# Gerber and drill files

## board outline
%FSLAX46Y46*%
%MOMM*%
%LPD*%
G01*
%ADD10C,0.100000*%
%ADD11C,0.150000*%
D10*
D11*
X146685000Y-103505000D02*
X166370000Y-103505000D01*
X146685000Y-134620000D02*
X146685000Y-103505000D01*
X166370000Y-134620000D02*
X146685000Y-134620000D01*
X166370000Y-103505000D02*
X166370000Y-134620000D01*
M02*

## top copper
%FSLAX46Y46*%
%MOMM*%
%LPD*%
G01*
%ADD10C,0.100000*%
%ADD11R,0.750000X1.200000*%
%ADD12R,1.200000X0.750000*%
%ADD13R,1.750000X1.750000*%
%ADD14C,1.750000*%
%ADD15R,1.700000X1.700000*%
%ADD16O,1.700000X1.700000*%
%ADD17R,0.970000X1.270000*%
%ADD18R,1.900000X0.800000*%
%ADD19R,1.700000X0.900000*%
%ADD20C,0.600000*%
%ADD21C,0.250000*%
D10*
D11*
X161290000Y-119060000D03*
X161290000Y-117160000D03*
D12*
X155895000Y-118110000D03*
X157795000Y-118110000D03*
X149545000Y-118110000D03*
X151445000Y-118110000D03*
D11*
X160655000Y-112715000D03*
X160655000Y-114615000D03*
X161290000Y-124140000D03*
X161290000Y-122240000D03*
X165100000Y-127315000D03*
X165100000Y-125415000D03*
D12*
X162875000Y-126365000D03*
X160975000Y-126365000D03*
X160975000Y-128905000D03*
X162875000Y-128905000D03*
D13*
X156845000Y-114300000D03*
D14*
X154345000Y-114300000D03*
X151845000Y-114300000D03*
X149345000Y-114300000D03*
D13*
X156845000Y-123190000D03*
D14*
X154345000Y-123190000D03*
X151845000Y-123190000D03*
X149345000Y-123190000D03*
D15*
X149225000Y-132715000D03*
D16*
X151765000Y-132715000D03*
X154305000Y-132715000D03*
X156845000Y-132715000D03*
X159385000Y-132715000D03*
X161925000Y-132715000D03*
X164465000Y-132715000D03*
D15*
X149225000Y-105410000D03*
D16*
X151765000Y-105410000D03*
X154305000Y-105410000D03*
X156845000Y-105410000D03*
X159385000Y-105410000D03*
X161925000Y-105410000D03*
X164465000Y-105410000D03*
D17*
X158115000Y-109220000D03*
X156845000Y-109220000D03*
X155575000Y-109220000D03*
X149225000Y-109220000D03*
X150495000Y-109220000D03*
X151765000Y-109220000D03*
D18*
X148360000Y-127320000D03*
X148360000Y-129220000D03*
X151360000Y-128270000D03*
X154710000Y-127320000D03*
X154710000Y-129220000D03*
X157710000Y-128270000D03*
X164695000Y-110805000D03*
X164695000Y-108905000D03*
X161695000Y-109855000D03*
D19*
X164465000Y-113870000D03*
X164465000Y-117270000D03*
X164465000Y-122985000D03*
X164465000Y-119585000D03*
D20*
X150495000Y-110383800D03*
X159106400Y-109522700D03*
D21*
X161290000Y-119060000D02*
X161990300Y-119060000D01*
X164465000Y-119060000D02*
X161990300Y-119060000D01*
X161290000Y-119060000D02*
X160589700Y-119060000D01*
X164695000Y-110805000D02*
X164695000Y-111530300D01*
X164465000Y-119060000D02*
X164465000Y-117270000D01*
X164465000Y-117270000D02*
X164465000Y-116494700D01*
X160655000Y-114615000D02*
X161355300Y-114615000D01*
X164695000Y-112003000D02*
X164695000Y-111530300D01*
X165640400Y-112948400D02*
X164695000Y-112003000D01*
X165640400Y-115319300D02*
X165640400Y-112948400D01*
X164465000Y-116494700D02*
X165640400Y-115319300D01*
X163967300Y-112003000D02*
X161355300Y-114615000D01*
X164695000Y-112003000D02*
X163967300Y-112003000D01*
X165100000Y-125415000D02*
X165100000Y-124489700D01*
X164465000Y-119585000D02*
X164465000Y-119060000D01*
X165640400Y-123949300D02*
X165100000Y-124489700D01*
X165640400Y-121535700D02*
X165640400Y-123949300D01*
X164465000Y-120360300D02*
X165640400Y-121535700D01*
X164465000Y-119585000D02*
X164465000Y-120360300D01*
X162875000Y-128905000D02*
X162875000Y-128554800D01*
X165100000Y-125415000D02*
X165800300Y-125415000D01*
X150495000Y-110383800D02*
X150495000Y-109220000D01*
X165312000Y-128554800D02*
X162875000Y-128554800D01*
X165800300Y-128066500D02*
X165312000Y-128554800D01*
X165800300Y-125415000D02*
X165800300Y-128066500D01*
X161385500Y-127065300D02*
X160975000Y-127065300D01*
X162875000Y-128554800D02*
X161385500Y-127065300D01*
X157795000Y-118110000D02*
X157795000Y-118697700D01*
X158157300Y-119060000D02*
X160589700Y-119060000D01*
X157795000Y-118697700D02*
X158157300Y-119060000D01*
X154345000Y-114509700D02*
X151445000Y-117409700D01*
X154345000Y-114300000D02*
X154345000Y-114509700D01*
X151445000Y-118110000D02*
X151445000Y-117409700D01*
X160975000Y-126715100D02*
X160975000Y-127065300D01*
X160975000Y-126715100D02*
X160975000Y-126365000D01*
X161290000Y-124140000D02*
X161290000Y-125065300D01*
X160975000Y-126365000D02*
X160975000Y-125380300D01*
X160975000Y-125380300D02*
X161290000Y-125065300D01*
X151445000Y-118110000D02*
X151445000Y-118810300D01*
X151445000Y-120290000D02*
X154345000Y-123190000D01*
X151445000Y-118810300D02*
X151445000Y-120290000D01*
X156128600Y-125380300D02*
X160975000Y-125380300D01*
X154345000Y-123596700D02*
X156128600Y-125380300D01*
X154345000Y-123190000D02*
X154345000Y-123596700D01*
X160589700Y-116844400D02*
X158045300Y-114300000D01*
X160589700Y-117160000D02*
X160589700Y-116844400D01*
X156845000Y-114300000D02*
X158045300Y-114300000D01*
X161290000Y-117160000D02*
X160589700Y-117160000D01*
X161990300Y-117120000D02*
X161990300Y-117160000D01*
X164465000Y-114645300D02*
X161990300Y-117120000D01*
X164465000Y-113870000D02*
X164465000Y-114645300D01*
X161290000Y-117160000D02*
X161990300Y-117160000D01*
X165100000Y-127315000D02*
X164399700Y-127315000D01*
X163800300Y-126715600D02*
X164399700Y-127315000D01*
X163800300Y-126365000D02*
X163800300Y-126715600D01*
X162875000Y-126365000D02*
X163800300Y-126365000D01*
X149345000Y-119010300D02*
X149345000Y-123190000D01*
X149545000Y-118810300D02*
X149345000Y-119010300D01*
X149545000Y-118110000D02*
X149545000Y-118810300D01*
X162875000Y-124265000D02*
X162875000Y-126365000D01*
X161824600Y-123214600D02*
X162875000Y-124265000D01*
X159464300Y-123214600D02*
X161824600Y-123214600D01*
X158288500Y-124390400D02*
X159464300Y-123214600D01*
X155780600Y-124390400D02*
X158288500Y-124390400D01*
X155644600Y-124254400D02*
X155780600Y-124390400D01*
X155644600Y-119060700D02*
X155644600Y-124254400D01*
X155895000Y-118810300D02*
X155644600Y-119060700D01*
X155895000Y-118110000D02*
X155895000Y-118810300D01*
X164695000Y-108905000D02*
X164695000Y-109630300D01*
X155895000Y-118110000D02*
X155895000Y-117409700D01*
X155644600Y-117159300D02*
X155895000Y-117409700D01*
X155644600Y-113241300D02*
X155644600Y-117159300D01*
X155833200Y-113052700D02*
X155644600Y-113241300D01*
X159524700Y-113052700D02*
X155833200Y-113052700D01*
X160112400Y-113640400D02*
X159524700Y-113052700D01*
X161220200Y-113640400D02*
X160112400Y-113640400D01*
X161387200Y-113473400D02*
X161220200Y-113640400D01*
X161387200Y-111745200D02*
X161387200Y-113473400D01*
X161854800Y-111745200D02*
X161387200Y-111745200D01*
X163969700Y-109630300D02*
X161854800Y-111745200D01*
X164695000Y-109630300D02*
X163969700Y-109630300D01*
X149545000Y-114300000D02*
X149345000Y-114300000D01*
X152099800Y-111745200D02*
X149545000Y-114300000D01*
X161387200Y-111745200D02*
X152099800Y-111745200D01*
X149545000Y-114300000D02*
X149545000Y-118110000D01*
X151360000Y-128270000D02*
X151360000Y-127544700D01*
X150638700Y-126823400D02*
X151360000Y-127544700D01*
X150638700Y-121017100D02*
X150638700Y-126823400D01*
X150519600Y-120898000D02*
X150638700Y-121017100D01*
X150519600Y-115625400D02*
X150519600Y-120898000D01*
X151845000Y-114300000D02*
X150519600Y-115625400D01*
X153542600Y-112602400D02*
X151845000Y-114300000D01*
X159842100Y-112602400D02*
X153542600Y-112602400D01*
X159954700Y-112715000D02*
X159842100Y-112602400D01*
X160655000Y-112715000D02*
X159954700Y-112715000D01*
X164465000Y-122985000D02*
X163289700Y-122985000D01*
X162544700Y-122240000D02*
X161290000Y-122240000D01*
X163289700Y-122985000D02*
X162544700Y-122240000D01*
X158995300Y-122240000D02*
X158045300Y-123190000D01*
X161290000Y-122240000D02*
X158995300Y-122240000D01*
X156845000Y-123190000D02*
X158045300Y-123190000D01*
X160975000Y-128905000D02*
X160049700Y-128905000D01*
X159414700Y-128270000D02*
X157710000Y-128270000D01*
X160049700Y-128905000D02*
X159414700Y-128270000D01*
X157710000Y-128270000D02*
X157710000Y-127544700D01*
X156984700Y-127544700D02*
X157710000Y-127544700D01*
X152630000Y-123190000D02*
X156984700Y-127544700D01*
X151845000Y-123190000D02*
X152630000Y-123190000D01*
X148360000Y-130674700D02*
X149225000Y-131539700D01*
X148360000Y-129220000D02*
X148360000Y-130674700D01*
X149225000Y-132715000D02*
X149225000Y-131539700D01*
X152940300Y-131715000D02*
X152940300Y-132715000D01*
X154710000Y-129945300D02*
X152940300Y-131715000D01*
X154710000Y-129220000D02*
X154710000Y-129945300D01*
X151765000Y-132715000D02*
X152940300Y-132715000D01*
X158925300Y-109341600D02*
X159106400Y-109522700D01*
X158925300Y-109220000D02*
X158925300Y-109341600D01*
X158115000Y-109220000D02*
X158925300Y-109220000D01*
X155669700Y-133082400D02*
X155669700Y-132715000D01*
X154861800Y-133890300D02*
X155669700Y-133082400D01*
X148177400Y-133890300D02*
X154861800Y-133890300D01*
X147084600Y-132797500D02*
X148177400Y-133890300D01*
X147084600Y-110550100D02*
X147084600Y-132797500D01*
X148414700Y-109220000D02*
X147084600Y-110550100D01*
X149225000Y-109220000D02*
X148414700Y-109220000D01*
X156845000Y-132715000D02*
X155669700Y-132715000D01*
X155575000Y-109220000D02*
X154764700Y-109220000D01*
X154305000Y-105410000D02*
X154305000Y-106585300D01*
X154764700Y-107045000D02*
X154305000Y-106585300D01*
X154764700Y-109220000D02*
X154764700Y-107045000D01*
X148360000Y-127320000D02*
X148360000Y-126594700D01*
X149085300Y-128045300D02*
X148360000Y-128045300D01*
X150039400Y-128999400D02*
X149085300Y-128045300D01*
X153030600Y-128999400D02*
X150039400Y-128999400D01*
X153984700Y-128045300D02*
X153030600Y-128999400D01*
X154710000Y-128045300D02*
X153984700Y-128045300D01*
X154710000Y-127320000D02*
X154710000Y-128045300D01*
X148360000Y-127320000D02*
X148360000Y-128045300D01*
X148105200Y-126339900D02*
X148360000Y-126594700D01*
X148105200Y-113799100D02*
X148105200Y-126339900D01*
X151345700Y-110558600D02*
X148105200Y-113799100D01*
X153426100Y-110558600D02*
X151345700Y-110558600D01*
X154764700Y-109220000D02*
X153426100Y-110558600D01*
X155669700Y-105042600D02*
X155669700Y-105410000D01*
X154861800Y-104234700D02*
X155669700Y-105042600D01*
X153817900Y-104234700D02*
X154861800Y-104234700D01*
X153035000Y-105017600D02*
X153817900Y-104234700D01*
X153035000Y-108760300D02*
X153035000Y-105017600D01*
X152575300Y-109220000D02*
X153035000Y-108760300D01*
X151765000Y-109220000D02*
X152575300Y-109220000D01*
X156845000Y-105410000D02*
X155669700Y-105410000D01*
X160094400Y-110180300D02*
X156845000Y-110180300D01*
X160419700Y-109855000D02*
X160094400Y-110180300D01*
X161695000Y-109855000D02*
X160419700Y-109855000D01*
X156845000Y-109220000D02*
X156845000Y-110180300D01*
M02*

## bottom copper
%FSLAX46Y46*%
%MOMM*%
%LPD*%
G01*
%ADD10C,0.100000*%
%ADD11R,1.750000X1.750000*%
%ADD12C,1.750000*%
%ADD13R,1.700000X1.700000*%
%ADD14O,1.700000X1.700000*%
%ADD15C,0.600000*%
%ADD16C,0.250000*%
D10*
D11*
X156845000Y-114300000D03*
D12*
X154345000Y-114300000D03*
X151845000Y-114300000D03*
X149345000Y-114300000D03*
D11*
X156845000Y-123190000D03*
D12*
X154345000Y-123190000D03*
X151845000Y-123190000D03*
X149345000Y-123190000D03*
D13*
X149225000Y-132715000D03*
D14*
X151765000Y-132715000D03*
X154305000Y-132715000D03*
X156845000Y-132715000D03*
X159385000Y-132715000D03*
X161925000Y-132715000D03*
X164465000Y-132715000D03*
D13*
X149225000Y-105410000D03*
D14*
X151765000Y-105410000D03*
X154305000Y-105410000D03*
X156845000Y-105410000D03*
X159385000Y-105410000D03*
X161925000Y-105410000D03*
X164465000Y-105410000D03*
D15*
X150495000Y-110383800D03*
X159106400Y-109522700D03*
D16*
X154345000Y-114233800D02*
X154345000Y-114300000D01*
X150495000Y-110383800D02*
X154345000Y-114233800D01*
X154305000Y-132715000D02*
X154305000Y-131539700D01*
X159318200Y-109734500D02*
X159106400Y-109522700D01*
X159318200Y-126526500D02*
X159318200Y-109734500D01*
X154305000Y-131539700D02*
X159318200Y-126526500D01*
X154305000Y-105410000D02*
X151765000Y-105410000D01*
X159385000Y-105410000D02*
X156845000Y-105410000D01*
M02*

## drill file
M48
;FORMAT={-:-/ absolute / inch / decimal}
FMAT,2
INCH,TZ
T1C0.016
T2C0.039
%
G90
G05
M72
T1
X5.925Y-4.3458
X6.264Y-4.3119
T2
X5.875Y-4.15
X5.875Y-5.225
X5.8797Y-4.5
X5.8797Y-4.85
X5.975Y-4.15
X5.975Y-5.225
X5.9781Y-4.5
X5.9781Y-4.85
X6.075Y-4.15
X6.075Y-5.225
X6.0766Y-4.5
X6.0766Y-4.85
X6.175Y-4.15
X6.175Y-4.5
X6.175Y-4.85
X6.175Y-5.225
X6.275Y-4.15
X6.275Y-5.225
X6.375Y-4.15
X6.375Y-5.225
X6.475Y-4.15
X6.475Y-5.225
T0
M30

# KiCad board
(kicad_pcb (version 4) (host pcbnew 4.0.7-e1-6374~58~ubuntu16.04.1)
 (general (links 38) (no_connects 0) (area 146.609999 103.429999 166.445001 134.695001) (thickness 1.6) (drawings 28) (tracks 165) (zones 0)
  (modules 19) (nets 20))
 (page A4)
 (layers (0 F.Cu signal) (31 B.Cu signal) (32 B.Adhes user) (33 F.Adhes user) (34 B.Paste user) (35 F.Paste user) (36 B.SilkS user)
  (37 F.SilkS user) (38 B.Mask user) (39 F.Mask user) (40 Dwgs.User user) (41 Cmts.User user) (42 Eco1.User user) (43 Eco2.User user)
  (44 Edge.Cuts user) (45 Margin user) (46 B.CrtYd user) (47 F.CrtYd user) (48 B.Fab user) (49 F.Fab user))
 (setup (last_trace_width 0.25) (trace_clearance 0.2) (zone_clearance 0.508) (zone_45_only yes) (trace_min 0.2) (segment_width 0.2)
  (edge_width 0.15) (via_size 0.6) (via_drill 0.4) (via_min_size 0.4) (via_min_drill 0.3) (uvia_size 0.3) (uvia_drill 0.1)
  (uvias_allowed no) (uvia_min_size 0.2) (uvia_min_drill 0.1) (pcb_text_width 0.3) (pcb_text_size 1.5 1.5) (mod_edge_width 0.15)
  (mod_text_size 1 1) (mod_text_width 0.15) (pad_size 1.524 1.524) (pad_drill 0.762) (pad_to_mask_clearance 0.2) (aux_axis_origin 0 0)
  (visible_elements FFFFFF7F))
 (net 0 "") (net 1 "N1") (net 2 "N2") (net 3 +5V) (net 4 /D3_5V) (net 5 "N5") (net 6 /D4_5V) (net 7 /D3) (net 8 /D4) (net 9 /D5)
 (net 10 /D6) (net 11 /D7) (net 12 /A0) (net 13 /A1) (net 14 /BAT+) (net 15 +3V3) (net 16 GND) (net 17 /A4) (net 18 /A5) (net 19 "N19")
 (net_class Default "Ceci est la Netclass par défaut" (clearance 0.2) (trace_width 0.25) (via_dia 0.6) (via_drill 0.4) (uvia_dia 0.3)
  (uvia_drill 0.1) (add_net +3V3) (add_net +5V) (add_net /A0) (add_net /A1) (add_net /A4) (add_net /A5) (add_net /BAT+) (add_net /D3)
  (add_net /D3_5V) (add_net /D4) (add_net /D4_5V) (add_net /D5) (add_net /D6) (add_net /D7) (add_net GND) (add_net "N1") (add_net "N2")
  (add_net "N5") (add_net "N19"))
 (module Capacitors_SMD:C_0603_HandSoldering (layer F.Cu) (at 161.29 118.11 90)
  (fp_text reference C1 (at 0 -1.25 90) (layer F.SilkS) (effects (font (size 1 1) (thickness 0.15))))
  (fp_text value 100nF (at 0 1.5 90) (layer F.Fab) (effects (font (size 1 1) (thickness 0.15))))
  (pad 1 smd rect (at -0.95 0 90) (size 1.2 0.75) (layers F.Cu F.Paste F.Mask) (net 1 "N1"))
  (pad 2 smd rect (at 0.95 0 90) (size 1.2 0.75) (layers F.Cu F.Paste F.Mask) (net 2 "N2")))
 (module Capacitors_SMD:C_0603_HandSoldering (layer F.Cu) (at 156.845 118.11)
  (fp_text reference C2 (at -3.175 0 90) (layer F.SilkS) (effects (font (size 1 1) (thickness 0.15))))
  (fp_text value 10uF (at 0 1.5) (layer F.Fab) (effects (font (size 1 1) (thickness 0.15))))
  (pad 1 smd rect (at -0.95 0) (size 1.2 0.75) (layers F.Cu F.Paste F.Mask) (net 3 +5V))
  (pad 2 smd rect (at 0.95 0) (size 1.2 0.75) (layers F.Cu F.Paste F.Mask) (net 1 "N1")))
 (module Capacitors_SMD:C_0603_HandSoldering (layer F.Cu) (at 150.495 118.11)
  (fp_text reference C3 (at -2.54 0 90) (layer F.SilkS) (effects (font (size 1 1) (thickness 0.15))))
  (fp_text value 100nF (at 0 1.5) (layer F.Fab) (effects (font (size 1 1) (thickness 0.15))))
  (pad 1 smd rect (at -0.95 0) (size 1.2 0.75) (layers F.Cu F.Paste F.Mask) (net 3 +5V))
  (pad 2 smd rect (at 0.95 0) (size 1.2 0.75) (layers F.Cu F.Paste F.Mask) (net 1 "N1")))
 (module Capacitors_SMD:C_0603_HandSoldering (layer F.Cu) (at 160.655 113.665 270)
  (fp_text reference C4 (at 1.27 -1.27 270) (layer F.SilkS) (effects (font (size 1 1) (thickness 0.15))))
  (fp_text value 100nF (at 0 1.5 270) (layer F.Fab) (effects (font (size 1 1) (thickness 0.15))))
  (pad 1 smd rect (at -0.95 0 270) (size 1.2 0.75) (layers F.Cu F.Paste F.Mask) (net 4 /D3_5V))
  (pad 2 smd rect (at 0.95 0 270) (size 1.2 0.75) (layers F.Cu F.Paste F.Mask) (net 1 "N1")))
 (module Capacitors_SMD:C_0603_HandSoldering (layer F.Cu) (at 161.29 123.19 90)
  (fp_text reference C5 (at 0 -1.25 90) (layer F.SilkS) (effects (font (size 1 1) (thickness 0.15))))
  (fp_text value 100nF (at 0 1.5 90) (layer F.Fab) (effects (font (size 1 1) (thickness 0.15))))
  (pad 1 smd rect (at -0.95 0 90) (size 1.2 0.75) (layers F.Cu F.Paste F.Mask) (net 1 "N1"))
  (pad 2 smd rect (at 0.95 0 90) (size 1.2 0.75) (layers F.Cu F.Paste F.Mask) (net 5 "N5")))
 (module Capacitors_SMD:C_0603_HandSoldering (layer F.Cu) (at 165.1 126.365 90)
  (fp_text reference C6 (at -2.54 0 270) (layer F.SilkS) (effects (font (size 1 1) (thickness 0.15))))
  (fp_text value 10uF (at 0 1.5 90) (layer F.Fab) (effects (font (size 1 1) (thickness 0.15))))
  (pad 1 smd rect (at -0.95 0 90) (size 1.2 0.75) (layers F.Cu F.Paste F.Mask) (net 3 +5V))
  (pad 2 smd rect (at 0.95 0 90) (size 1.2 0.75) (layers F.Cu F.Paste F.Mask) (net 1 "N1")))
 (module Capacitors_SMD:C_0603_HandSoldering (layer F.Cu) (at 161.925 126.365 180)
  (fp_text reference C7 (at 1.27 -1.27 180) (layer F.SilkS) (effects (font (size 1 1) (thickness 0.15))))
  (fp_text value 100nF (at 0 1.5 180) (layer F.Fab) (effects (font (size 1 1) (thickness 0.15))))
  (pad 1 smd rect (at -0.95 0 180) (size 1.2 0.75) (layers F.Cu F.Paste F.Mask) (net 3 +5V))
  (pad 2 smd rect (at 0.95 0 180) (size 1.2 0.75) (layers F.Cu F.Paste F.Mask) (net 1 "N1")))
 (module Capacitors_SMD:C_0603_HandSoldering (layer F.Cu) (at 161.925 128.905)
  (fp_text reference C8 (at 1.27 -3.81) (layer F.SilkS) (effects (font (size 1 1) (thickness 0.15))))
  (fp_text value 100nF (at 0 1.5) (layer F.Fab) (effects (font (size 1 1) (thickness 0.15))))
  (pad 1 smd rect (at -0.95 0) (size 1.2 0.75) (layers F.Cu F.Paste F.Mask) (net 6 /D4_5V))
  (pad 2 smd rect (at 0.95 0) (size 1.2 0.75) (layers F.Cu F.Paste F.Mask) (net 1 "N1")))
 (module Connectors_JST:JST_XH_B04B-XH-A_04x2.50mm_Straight (layer F.Cu) (at 156.845 114.3 180)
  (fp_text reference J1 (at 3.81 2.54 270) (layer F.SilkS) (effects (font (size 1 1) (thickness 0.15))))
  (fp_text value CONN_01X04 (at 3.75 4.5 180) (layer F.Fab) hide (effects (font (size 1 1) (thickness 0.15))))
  (pad 1 thru_hole rect (at 0 0 180) (size 1.75 1.75) (drill 1) (layers *.Cu *.Mask) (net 2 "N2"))
  (pad 2 thru_hole circle (at 2.5 0 180) (size 1.75 1.75) (drill 1) (layers *.Cu *.Mask) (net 1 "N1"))
  (pad 3 thru_hole circle (at 5 0 180) (size 1.75 1.75) (drill 1) (layers *.Cu *.Mask) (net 4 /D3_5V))
  (pad 4 thru_hole circle (at 7.5 0 180) (size 1.75 1.75) (drill 1) (layers *.Cu *.Mask) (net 3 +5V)))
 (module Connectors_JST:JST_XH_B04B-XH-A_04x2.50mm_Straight (layer F.Cu) (at 156.845 123.19 180)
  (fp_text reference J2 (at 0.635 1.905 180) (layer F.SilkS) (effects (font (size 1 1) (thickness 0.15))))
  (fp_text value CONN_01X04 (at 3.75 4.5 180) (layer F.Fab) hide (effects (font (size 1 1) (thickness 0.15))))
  (pad 1 thru_hole rect (at 0 0 180) (size 1.75 1.75) (drill 1) (layers *.Cu *.Mask) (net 5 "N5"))
  (pad 2 thru_hole circle (at 2.5 0 180) (size 1.75 1.75) (drill 1) (layers *.Cu *.Mask) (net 1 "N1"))
  (pad 3 thru_hole circle (at 5 0 180) (size 1.75 1.75) (drill 1) (layers *.Cu *.Mask) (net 6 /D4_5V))
  (pad 4 thru_hole circle (at 7.5 0 180) (size 1.75 1.75) (drill 1) (layers *.Cu *.Mask) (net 3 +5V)))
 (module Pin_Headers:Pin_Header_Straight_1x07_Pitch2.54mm (layer B.Cu) (at 149.225 132.715 270)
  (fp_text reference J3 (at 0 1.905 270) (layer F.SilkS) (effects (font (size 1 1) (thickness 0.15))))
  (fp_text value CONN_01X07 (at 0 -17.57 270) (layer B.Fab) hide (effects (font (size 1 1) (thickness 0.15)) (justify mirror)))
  (pad 1 thru_hole rect (at 0 0 270) (size 1.7 1.7) (drill 1) (layers *.Cu *.Mask) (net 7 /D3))
  (pad 2 thru_hole oval (at 0 -2.54 270) (size 1.7 1.7) (drill 1) (layers *.Cu *.Mask) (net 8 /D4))
  (pad 3 thru_hole oval (at 0 -5.08 270) (size 1.7 1.7) (drill 1) (layers *.Cu *.Mask) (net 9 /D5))
  (pad 4 thru_hole oval (at 0 -7.62 270) (size 1.7 1.7) (drill 1) (layers *.Cu *.Mask) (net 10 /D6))
  (pad 5 thru_hole oval (at 0 -10.16 270) (size 1.7 1.7) (drill 1) (layers *.Cu *.Mask) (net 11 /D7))
  (pad 6 thru_hole oval (at 0 -12.7 270) (size 1.7 1.7) (drill 1) (layers *.Cu *.Mask) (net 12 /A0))
  (pad 7 thru_hole oval (at 0 -15.24 270) (size 1.7 1.7) (drill 1) (layers *.Cu *.Mask) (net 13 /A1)))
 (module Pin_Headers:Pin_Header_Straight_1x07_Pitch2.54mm (layer B.Cu) (at 149.225 105.41 270)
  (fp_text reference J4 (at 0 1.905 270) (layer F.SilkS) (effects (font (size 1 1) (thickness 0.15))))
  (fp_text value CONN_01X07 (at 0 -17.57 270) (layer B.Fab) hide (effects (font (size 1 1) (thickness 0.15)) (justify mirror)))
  (pad 1 thru_hole rect (at 0 0 270) (size 1.7 1.7) (drill 1) (layers *.Cu *.Mask) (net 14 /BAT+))
  (pad 2 thru_hole oval (at 0 -2.54 270) (size 1.7 1.7) (drill 1) (layers *.Cu *.Mask) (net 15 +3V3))
  (pad 3 thru_hole oval (at 0 -5.08 270) (size 1.7 1.7) (drill 1) (layers *.Cu *.Mask) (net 15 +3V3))
  (pad 4 thru_hole oval (at 0 -7.62 270) (size 1.7 1.7) (drill 1) (layers *.Cu *.Mask) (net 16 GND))
  (pad 5 thru_hole oval (at 0 -10.16 270) (size 1.7 1.7) (drill 1) (layers *.Cu *.Mask) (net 16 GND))
  (pad 6 thru_hole oval (at 0 -12.7 270) (size 1.7 1.7) (drill 1) (layers *.Cu *.Mask) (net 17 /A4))
  (pad 7 thru_hole oval (at 0 -15.24 270) (size 1.7 1.7) (drill 1) (layers *.Cu *.Mask) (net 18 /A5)))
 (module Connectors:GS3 (layer F.Cu) (at 156.845 109.22 270)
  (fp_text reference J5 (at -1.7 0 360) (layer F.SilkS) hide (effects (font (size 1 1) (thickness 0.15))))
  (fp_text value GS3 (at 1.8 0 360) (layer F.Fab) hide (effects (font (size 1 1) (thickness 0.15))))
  (pad 1 smd rect (at 0 -1.27 270) (size 1.27 0.97) (layers F.Cu F.Paste F.Mask) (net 9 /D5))
  (pad 2 smd rect (at 0 0 270) (size 1.27 0.97) (layers F.Cu F.Paste F.Mask) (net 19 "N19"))
  (pad 3 smd rect (at 0 1.27 270) (size 1.27 0.97) (layers F.Cu F.Paste F.Mask) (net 15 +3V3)))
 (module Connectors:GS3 (layer F.Cu) (at 150.495 109.22 90)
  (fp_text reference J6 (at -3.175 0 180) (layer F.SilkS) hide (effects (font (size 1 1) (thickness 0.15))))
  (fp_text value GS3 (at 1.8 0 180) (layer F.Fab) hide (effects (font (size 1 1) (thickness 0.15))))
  (pad 1 smd rect (at 0 -1.27 90) (size 1.27 0.97) (layers F.Cu F.Paste F.Mask) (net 10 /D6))
  (pad 2 smd rect (at 0 0 90) (size 1.27 0.97) (layers F.Cu F.Paste F.Mask) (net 1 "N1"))
  (pad 3 smd rect (at 0 1.27 90) (size 1.27 0.97) (layers F.Cu F.Paste F.Mask) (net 16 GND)))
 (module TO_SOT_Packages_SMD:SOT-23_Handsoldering (layer F.Cu) (at 149.86 128.27)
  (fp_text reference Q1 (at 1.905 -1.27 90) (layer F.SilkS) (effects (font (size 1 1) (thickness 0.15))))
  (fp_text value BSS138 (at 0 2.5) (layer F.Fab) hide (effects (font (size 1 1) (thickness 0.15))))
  (pad 1 smd rect (at -1.5 -0.95) (size 1.9 0.8) (layers F.Cu F.Paste F.Mask) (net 15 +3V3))
  (pad 2 smd rect (at -1.5 0.95) (size 1.9 0.8) (layers F.Cu F.Paste F.Mask) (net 7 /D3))
  (pad 3 smd rect (at 1.5 0) (size 1.9 0.8) (layers F.Cu F.Paste F.Mask) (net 4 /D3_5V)))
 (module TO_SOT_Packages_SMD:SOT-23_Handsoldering (layer F.Cu) (at 156.21 128.27)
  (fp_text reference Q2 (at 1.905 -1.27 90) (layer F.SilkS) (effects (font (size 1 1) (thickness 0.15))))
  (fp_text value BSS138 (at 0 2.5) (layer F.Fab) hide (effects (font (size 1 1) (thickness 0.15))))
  (pad 1 smd rect (at -1.5 -0.95) (size 1.9 0.8) (layers F.Cu F.Paste F.Mask) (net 15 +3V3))
  (pad 2 smd rect (at -1.5 0.95) (size 1.9 0.8) (layers F.Cu F.Paste F.Mask) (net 8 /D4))
  (pad 3 smd rect (at 1.5 0) (size 1.9 0.8) (layers F.Cu F.Paste F.Mask) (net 6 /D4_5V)))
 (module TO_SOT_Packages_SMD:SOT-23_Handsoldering (layer F.Cu) (at 163.195 109.855 180)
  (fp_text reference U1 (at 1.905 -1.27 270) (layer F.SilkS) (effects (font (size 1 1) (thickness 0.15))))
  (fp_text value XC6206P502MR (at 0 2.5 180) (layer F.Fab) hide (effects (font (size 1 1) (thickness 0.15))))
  (pad 1 smd rect (at -1.5 -0.95 180) (size 1.9 0.8) (layers F.Cu F.Paste F.Mask) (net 1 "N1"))
  (pad 2 smd rect (at -1.5 0.95 180) (size 1.9 0.8) (layers F.Cu F.Paste F.Mask) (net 3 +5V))
  (pad 3 smd rect (at 1.5 0 180) (size 1.9 0.8) (layers F.Cu F.Paste F.Mask) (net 19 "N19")))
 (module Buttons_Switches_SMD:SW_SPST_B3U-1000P (layer F.Cu) (at 164.465 115.57 270)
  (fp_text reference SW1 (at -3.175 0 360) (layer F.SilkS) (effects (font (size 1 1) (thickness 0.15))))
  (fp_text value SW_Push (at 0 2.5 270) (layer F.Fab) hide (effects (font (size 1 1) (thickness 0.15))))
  (pad 1 smd rect (at -1.7 0 270) (size 0.9 1.7) (layers F.Cu F.Paste F.Mask) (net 2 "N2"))
  (pad 2 smd rect (at 1.7 0 270) (size 0.9 1.7) (layers F.Cu F.Paste F.Mask) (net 1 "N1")))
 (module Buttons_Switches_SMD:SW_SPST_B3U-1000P (layer F.Cu) (at 164.465 121.285 90)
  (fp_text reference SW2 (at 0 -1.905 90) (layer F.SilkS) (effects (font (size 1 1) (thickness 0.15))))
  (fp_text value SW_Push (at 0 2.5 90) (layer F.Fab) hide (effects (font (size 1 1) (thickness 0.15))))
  (pad 1 smd rect (at -1.7 0 90) (size 0.9 1.7) (layers F.Cu F.Paste F.Mask) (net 5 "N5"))
  (pad 2 smd rect (at 1.7 0 90) (size 0.9 1.7) (layers F.Cu F.Paste F.Mask) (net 1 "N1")))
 (gr_line (start 146.685 103.505) (end 166.37 103.505) (angle 90) (layer Edge.Cuts) (width 0.15))
 (gr_line (start 146.685 134.62) (end 146.685 103.505) (angle 90) (layer Edge.Cuts) (width 0.15))
 (gr_line (start 166.37 134.62) (end 146.685 134.62) (angle 90) (layer Edge.Cuts) (width 0.15))
 (gr_line (start 166.37 103.505) (end 166.37 134.62) (angle 90) (layer Edge.Cuts) (width 0.15))
 (via (at 150.495 110.3838) (size 0.6) (layers F.Cu B.Cu) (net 1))
 (segment (start 161.29 119.06) (end 161.9903 119.06) (width 0.25) (layer F.Cu) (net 1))
 (segment (start 164.465 119.06) (end 161.9903 119.06) (width 0.25) (layer F.Cu) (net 1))
 (segment (start 161.29 119.06) (end 160.5897 119.06) (width 0.25) (layer F.Cu) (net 1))
 (segment (start 164.695 110.805) (end 164.695 111.5303) (width 0.25) (layer F.Cu) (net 1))
 (segment (start 164.465 119.06) (end 164.465 117.27) (width 0.25) (layer F.Cu) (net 1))
 (segment (start 164.465 117.27) (end 164.465 116.4947) (width 0.25) (layer F.Cu) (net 1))
 (segment (start 160.655 114.615) (end 161.3553 114.615) (width 0.25) (layer F.Cu) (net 1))
 (segment (start 164.695 112.003) (end 164.695 111.5303) (width 0.25) (layer F.Cu) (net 1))
 (segment (start 165.6404 112.9484) (end 164.695 112.003) (width 0.25) (layer F.Cu) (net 1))
 (segment (start 165.6404 115.3193) (end 165.6404 112.9484) (width 0.25) (layer F.Cu) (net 1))
 (segment (start 164.465 116.4947) (end 165.6404 115.3193) (width 0.25) (layer F.Cu) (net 1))
 (segment (start 163.9673 112.003) (end 161.3553 114.615) (width 0.25) (layer F.Cu) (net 1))
 (segment (start 164.695 112.003) (end 163.9673 112.003) (width 0.25) (layer F.Cu) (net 1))
 (segment (start 165.1 125.415) (end 165.1 124.4897) (width 0.25) (layer F.Cu) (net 1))
 (segment (start 164.465 119.585) (end 164.465 119.06) (width 0.25) (layer F.Cu) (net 1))
 (segment (start 165.6404 123.9493) (end 165.1 124.4897) (width 0.25) (layer F.Cu) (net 1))
 (segment (start 165.6404 121.5357) (end 165.6404 123.9493) (width 0.25) (layer F.Cu) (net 1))
 (segment (start 164.465 120.3603) (end 165.6404 121.5357) (width 0.25) (layer F.Cu) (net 1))
 (segment (start 164.465 119.585) (end 164.465 120.3603) (width 0.25) (layer F.Cu) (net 1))
 (segment (start 162.875 128.905) (end 162.875 128.5548) (width 0.25) (layer F.Cu) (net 1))
 (segment (start 165.1 125.415) (end 165.8003 125.415) (width 0.25) (layer F.Cu) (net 1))
 (segment (start 150.495 110.3838) (end 150.495 109.22) (width 0.25) (layer F.Cu) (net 1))
 (segment (start 154.345 114.2338) (end 154.345 114.3) (width 0.25) (layer B.Cu) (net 1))
 (segment (start 150.495 110.3838) (end 154.345 114.2338) (width 0.25) (layer B.Cu) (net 1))
 (segment (start 165.312 128.5548) (end 162.875 128.5548) (width 0.25) (layer F.Cu) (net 1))
 (segment (start 165.8003 128.0665) (end 165.312 128.5548) (width 0.25) (layer F.Cu) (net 1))
 (segment (start 165.8003 125.415) (end 165.8003 128.0665) (width 0.25) (layer F.Cu) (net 1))
 (segment (start 161.3855 127.0653) (end 160.975 127.0653) (width 0.25) (layer F.Cu) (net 1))
 (segment (start 162.875 128.5548) (end 161.3855 127.0653) (width 0.25) (layer F.Cu) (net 1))
 (segment (start 157.795 118.11) (end 157.795 118.6977) (width 0.25) (layer F.Cu) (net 1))
 (segment (start 158.1573 119.06) (end 160.5897 119.06) (width 0.25) (layer F.Cu) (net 1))
 (segment (start 157.795 118.6977) (end 158.1573 119.06) (width 0.25) (layer F.Cu) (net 1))
 (segment (start 154.345 114.5097) (end 151.445 117.4097) (width 0.25) (layer F.Cu) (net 1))
 (segment (start 154.345 114.3) (end 154.345 114.5097) (width 0.25) (layer F.Cu) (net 1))
 (segment (start 151.445 118.11) (end 151.445 117.4097) (width 0.25) (layer F.Cu) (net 1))
 (segment (start 160.975 126.7151) (end 160.975 127.0653) (width 0.25) (layer F.Cu) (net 1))
 (segment (start 160.975 126.7151) (end 160.975 126.365) (width 0.25) (layer F.Cu) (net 1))
 (segment (start 161.29 124.14) (end 161.29 125.0653) (width 0.25) (layer F.Cu) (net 1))
 (segment (start 160.975 126.365) (end 160.975 125.3803) (width 0.25) (layer F.Cu) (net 1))
 (segment (start 160.975 125.3803) (end 161.29 125.0653) (width 0.25) (layer F.Cu) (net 1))
 (segment (start 151.445 118.11) (end 151.445 118.8103) (width 0.25) (layer F.Cu) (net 1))
 (segment (start 151.445 120.29) (end 154.345 123.19) (width 0.25) (layer F.Cu) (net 1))
 (segment (start 151.445 118.8103) (end 151.445 120.29) (width 0.25) (layer F.Cu) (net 1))
 (segment (start 156.1286 125.3803) (end 160.975 125.3803) (width 0.25) (layer F.Cu) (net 1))
 (segment (start 154.345 123.5967) (end 156.1286 125.3803) (width 0.25) (layer F.Cu) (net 1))
 (segment (start 154.345 123.19) (end 154.345 123.5967) (width 0.25) (layer F.Cu) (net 1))
 (segment (start 160.5897 116.8444) (end 158.0453 114.3) (width 0.25) (layer F.Cu) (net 2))
 (segment (start 160.5897 117.16) (end 160.5897 116.8444) (width 0.25) (layer F.Cu) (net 2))
 (segment (start 156.845 114.3) (end 158.0453 114.3) (width 0.25) (layer F.Cu) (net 2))
 (segment (start 161.29 117.16) (end 160.5897 117.16) (width 0.25) (layer F.Cu) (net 2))
 (segment (start 161.9903 117.12) (end 161.9903 117.16) (width 0.25) (layer F.Cu) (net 2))
 (segment (start 164.465 114.6453) (end 161.9903 117.12) (width 0.25) (layer F.Cu) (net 2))
 (segment (start 164.465 113.87) (end 164.465 114.6453) (width 0.25) (layer F.Cu) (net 2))
 (segment (start 161.29 117.16) (end 161.9903 117.16) (width 0.25) (layer F.Cu) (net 2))
 (segment (start 165.1 127.315) (end 164.3997 127.315) (width 0.25) (layer F.Cu) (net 3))
 (segment (start 163.8003 126.7156) (end 164.3997 127.315) (width 0.25) (layer F.Cu) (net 3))
 (segment (start 163.8003 126.365) (end 163.8003 126.7156) (width 0.25) (layer F.Cu) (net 3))
 (segment (start 162.875 126.365) (end 163.8003 126.365) (width 0.25) (layer F.Cu) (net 3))
 (segment (start 149.345 119.0103) (end 149.345 123.19) (width 0.25) (layer F.Cu) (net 3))
 (segment (start 149.545 118.8103) (end 149.345 119.0103) (width 0.25) (layer F.Cu) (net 3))
 (segment (start 149.545 118.11) (end 149.545 118.8103) (width 0.25) (layer F.Cu) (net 3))
 (segment (start 162.875 124.265) (end 162.875 126.365) (width 0.25) (layer F.Cu) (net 3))
 (segment (start 161.8246 123.2146) (end 162.875 124.265) (width 0.25) (layer F.Cu) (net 3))
 (segment (start 159.4643 123.2146) (end 161.8246 123.2146) (width 0.25) (layer F.Cu) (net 3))
 (segment (start 158.2885 124.3904) (end 159.4643 123.2146) (width 0.25) (layer F.Cu) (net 3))
 (segment (start 155.7806 124.3904) (end 158.2885 124.3904) (width 0.25) (layer F.Cu) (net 3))
 (segment (start 155.6446 124.2544) (end 155.7806 124.3904) (width 0.25) (layer F.Cu) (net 3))
 (segment (start 155.6446 119.0607) (end 155.6446 124.2544) (width 0.25) (layer F.Cu) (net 3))
 (segment (start 155.895 118.8103) (end 155.6446 119.0607) (width 0.25) (layer F.Cu) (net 3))
 (segment (start 155.895 118.11) (end 155.895 118.8103) (width 0.25) (layer F.Cu) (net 3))
 (segment (start 164.695 108.905) (end 164.695 109.6303) (width 0.25) (layer F.Cu) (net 3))
 (segment (start 155.895 118.11) (end 155.895 117.4097) (width 0.25) (layer F.Cu) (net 3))
 (segment (start 155.6446 117.1593) (end 155.895 117.4097) (width 0.25) (layer F.Cu) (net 3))
 (segment (start 155.6446 113.2413) (end 155.6446 117.1593) (width 0.25) (layer F.Cu) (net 3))
 (segment (start 155.8332 113.0527) (end 155.6446 113.2413) (width 0.25) (layer F.Cu) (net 3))
 (segment (start 159.5247 113.0527) (end 155.8332 113.0527) (width 0.25) (layer F.Cu) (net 3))
 (segment (start 160.1124 113.6404) (end 159.5247 113.0527) (width 0.25) (layer F.Cu) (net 3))
 (segment (start 161.2202 113.6404) (end 160.1124 113.6404) (width 0.25) (layer F.Cu) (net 3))
 (segment (start 161.3872 113.4734) (end 161.2202 113.6404) (width 0.25) (layer F.Cu) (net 3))
 (segment (start 161.3872 111.7452) (end 161.3872 113.4734) (width 0.25) (layer F.Cu) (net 3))
 (segment (start 161.8548 111.7452) (end 161.3872 111.7452) (width 0.25) (layer F.Cu) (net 3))
 (segment (start 163.9697 109.6303) (end 161.8548 111.7452) (width 0.25) (layer F.Cu) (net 3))
 (segment (start 164.695 109.6303) (end 163.9697 109.6303) (width 0.25) (layer F.Cu) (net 3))
 (segment (start 149.545 114.3) (end 149.345 114.3) (width 0.25) (layer F.Cu) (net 3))
 (segment (start 152.0998 111.7452) (end 149.545 114.3) (width 0.25) (layer F.Cu) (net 3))
 (segment (start 161.3872 111.7452) (end 152.0998 111.7452) (width 0.25) (layer F.Cu) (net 3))
 (segment (start 149.545 114.3) (end 149.545 118.11) (width 0.25) (layer F.Cu) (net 3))
 (segment (start 151.36 128.27) (end 151.36 127.5447) (width 0.25) (layer F.Cu) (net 4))
 (segment (start 150.6387 126.8234) (end 151.36 127.5447) (width 0.25) (layer F.Cu) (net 4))
 (segment (start 150.6387 121.0171) (end 150.6387 126.8234) (width 0.25) (layer F.Cu) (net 4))
 (segment (start 150.5196 120.898) (end 150.6387 121.0171) (width 0.25) (layer F.Cu) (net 4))
 (segment (start 150.5196 115.6254) (end 150.5196 120.898) (width 0.25) (layer F.Cu) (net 4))
 (segment (start 151.845 114.3) (end 150.5196 115.6254) (width 0.25) (layer F.Cu) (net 4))
 (segment (start 153.5426 112.6024) (end 151.845 114.3) (width 0.25) (layer F.Cu) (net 4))
 (segment (start 159.8421 112.6024) (end 153.5426 112.6024) (width 0.25) (layer F.Cu) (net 4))
 (segment (start 159.9547 112.715) (end 159.8421 112.6024) (width 0.25) (layer F.Cu) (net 4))
 (segment (start 160.655 112.715) (end 159.9547 112.715) (width 0.25) (layer F.Cu) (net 4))
 (segment (start 164.465 122.985) (end 163.2897 122.985) (width 0.25) (layer F.Cu) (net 5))
 (segment (start 162.5447 122.24) (end 161.29 122.24) (width 0.25) (layer F.Cu) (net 5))
 (segment (start 163.2897 122.985) (end 162.5447 122.24) (width 0.25) (layer F.Cu) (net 5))
 (segment (start 158.9953 122.24) (end 158.0453 123.19) (width 0.25) (layer F.Cu) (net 5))
 (segment (start 161.29 122.24) (end 158.9953 122.24) (width 0.25) (layer F.Cu) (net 5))
 (segment (start 156.845 123.19) (end 158.0453 123.19) (width 0.25) (layer F.Cu) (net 5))
 (segment (start 160.975 128.905) (end 160.0497 128.905) (width 0.25) (layer F.Cu) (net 6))
 (segment (start 159.4147 128.27) (end 157.71 128.27) (width 0.25) (layer F.Cu) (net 6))
 (segment (start 160.0497 128.905) (end 159.4147 128.27) (width 0.25) (layer F.Cu) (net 6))
 (segment (start 157.71 128.27) (end 157.71 127.5447) (width 0.25) (layer F.Cu) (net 6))
 (segment (start 156.9847 127.5447) (end 157.71 127.5447) (width 0.25) (layer F.Cu) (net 6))
 (segment (start 152.63 123.19) (end 156.9847 127.5447) (width 0.25) (layer F.Cu) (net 6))
 (segment (start 151.845 123.19) (end 152.63 123.19) (width 0.25) (layer F.Cu) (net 6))
 (segment (start 148.36 130.6747) (end 149.225 131.5397) (width 0.25) (layer F.Cu) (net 7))
 (segment (start 148.36 129.22) (end 148.36 130.6747) (width 0.25) (layer F.Cu) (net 7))
 (segment (start 149.225 132.715) (end 149.225 131.5397) (width 0.25) (layer F.Cu) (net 7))
 (segment (start 152.9403 131.715) (end 152.9403 132.715) (width 0.25) (layer F.Cu) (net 8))
 (segment (start 154.71 129.9453) (end 152.9403 131.715) (width 0.25) (layer F.Cu) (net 8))
 (segment (start 154.71 129.22) (end 154.71 129.9453) (width 0.25) (layer F.Cu) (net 8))
 (segment (start 151.765 132.715) (end 152.9403 132.715) (width 0.25) (layer F.Cu) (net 8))
 (via (at 159.1064 109.5227) (size 0.6) (layers F.Cu B.Cu) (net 9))
 (segment (start 158.9253 109.3416) (end 159.1064 109.5227) (width 0.25) (layer F.Cu) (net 9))
 (segment (start 158.9253 109.22) (end 158.9253 109.3416) (width 0.25) (layer F.Cu) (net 9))
 (segment (start 154.305 132.715) (end 154.305 131.5397) (width 0.25) (layer B.Cu) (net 9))
 (segment (start 158.115 109.22) (end 158.9253 109.22) (width 0.25) (layer F.Cu) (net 9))
 (segment (start 159.3182 109.7345) (end 159.1064 109.5227) (width 0.25) (layer B.Cu) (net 9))
 (segment (start 159.3182 126.5265) (end 159.3182 109.7345) (width 0.25) (layer B.Cu) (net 9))
 (segment (start 154.305 131.5397) (end 159.3182 126.5265) (width 0.25) (layer B.Cu) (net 9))
 (segment (start 155.6697 133.0824) (end 155.6697 132.715) (width 0.25) (layer F.Cu) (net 10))
 (segment (start 154.8618 133.8903) (end 155.6697 133.0824) (width 0.25) (layer F.Cu) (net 10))
 (segment (start 148.1774 133.8903) (end 154.8618 133.8903) (width 0.25) (layer F.Cu) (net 10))
 (segment (start 147.0846 132.7975) (end 148.1774 133.8903) (width 0.25) (layer F.Cu) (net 10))
 (segment (start 147.0846 110.5501) (end 147.0846 132.7975) (width 0.25) (layer F.Cu) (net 10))
 (segment (start 148.4147 109.22) (end 147.0846 110.5501) (width 0.25) (layer F.Cu) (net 10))
 (segment (start 149.225 109.22) (end 148.4147 109.22) (width 0.25) (layer F.Cu) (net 10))
 (segment (start 156.845 132.715) (end 155.6697 132.715) (width 0.25) (layer F.Cu) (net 10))
 (segment (start 155.575 109.22) (end 154.7647 109.22) (width 0.25) (layer F.Cu) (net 15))
 (segment (start 154.305 105.41) (end 154.305 106.5853) (width 0.25) (layer F.Cu) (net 15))
 (segment (start 154.305 105.41) (end 151.765 105.41) (width 0.25) (layer B.Cu) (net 15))
 (segment (start 154.7647 107.045) (end 154.305 106.5853) (width 0.25) (layer F.Cu) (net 15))
 (segment (start 154.7647 109.22) (end 154.7647 107.045) (width 0.25) (layer F.Cu) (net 15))
 (segment (start 148.36 127.32) (end 148.36 126.5947) (width 0.25) (layer F.Cu) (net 15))
 (segment (start 149.0853 128.0453) (end 148.36 128.0453) (width 0.25) (layer F.Cu) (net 15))
 (segment (start 150.0394 128.9994) (end 149.0853 128.0453) (width 0.25) (layer F.Cu) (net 15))
 (segment (start 153.0306 128.9994) (end 150.0394 128.9994) (width 0.25) (layer F.Cu) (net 15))
 (segment (start 153.9847 128.0453) (end 153.0306 128.9994) (width 0.25) (layer F.Cu) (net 15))
 (segment (start 154.71 128.0453) (end 153.9847 128.0453) (width 0.25) (layer F.Cu) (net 15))
 (segment (start 154.71 127.32) (end 154.71 128.0453) (width 0.25) (layer F.Cu) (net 15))
 (segment (start 148.36 127.32) (end 148.36 128.0453) (width 0.25) (layer F.Cu) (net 15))
 (segment (start 148.1052 126.3399) (end 148.36 126.5947) (width 0.25) (layer F.Cu) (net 15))
 (segment (start 148.1052 113.7991) (end 148.1052 126.3399) (width 0.25) (layer F.Cu) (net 15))
 (segment (start 151.3457 110.5586) (end 148.1052 113.7991) (width 0.25) (layer F.Cu) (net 15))
 (segment (start 153.4261 110.5586) (end 151.3457 110.5586) (width 0.25) (layer F.Cu) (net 15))
 (segment (start 154.7647 109.22) (end 153.4261 110.5586) (width 0.25) (layer F.Cu) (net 15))
 (segment (start 159.385 105.41) (end 156.845 105.41) (width 0.25) (layer B.Cu) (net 16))
 (segment (start 155.6697 105.0426) (end 155.6697 105.41) (width 0.25) (layer F.Cu) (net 16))
 (segment (start 154.8618 104.2347) (end 155.6697 105.0426) (width 0.25) (layer F.Cu) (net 16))
 (segment (start 153.8179 104.2347) (end 154.8618 104.2347) (width 0.25) (layer F.Cu) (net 16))
 (segment (start 153.035 105.0176) (end 153.8179 104.2347) (width 0.25) (layer F.Cu) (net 16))
 (segment (start 153.035 108.7603) (end 153.035 105.0176) (width 0.25) (layer F.Cu) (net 16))
 (segment (start 152.5753 109.22) (end 153.035 108.7603) (width 0.25) (layer F.Cu) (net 16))
 (segment (start 151.765 109.22) (end 152.5753 109.22) (width 0.25) (layer F.Cu) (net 16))
 (segment (start 156.845 105.41) (end 155.6697 105.41) (width 0.25) (layer F.Cu) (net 16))
 (segment (start 160.0944 110.1803) (end 156.845 110.1803) (width 0.25) (layer F.Cu) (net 19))
 (segment (start 160.4197 109.855) (end 160.0944 110.1803) (width 0.25) (layer F.Cu) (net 19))
 (segment (start 161.695 109.855) (end 160.4197 109.855) (width 0.25) (layer F.Cu) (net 19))
 (segment (start 156.845 109.22) (end 156.845 110.1803) (width 0.25) (layer F.Cu) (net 19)))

